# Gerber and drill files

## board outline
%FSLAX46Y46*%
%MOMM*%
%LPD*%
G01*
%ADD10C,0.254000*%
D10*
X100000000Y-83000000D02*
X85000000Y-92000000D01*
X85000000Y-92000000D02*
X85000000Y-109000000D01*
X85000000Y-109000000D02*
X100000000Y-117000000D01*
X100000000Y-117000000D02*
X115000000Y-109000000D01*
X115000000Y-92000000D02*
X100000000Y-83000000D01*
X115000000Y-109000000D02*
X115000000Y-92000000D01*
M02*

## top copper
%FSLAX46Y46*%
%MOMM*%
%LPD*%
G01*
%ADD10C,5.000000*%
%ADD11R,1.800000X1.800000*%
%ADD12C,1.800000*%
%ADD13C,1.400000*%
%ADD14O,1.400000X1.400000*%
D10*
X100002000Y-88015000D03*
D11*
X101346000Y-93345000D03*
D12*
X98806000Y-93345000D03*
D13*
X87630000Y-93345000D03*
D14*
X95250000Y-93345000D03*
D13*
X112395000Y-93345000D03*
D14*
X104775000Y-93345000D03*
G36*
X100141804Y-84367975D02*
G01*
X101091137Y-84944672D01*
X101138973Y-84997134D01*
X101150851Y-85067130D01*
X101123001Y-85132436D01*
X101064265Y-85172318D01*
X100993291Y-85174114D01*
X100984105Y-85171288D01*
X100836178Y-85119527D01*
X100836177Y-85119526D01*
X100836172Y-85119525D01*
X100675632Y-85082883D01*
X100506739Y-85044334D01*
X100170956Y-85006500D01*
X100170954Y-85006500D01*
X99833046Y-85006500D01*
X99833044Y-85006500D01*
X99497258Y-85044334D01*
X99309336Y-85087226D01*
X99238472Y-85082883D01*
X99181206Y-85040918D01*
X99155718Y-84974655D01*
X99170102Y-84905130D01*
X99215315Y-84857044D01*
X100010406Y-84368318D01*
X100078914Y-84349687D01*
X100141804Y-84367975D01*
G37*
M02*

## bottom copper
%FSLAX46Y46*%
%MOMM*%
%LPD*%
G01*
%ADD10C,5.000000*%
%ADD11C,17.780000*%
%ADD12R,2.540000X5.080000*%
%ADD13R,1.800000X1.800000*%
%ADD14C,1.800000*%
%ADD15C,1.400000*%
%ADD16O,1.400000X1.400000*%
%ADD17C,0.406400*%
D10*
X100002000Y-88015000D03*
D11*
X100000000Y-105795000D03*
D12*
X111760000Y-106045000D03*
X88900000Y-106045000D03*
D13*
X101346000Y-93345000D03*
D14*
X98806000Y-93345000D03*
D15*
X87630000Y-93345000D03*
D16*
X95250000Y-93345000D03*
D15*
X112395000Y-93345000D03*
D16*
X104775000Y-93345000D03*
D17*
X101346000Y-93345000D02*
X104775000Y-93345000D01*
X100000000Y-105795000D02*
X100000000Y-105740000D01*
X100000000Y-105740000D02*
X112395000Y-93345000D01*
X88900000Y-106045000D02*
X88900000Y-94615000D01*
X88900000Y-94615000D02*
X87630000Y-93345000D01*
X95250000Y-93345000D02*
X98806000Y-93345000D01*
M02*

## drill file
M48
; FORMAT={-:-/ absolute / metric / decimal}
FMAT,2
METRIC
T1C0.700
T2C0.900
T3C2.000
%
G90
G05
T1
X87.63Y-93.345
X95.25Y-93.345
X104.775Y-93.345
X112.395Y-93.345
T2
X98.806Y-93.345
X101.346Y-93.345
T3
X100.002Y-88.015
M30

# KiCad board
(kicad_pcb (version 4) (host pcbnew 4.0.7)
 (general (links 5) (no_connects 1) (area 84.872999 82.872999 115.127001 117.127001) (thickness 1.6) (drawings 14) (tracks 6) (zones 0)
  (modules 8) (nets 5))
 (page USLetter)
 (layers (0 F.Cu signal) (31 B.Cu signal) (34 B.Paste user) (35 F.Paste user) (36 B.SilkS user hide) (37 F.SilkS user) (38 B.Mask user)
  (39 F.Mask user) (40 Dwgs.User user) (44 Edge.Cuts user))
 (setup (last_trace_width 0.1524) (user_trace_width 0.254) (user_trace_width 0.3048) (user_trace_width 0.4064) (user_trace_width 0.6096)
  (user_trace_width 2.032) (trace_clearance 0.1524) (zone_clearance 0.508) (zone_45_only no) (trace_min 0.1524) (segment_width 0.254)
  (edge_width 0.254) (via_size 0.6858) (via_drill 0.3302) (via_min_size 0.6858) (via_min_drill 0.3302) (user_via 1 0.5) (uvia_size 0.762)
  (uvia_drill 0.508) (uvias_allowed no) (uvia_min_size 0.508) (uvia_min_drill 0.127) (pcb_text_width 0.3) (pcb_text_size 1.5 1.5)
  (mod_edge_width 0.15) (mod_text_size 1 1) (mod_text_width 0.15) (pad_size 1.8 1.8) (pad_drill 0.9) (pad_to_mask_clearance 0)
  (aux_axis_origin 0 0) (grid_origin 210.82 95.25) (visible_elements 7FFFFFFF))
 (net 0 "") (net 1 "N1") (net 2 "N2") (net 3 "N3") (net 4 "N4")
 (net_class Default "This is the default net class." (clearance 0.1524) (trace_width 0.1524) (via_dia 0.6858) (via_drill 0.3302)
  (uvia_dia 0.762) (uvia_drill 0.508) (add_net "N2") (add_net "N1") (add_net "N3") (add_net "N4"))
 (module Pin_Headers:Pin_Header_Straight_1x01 (layer F.Cu) (at 99.822 88.265)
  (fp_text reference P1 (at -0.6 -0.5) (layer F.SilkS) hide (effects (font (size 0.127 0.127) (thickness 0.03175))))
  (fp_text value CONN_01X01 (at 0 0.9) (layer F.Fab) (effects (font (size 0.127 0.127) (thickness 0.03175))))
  (pad "" thru_hole circle (at 0.18 -0.25) (size 5 5) (drill 2) (layers *.Cu B.Mask)))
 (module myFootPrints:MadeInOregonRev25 (layer F.Cu) (at 108.585 93.091)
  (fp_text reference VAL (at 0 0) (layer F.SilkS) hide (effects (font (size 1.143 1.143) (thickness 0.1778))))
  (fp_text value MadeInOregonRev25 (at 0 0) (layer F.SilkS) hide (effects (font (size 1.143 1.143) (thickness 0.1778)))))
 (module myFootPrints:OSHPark (layer F.Cu) (at 99.949 99.822)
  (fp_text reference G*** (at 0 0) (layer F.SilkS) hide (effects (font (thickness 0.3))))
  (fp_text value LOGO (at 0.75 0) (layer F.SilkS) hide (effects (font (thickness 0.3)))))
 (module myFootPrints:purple (layer F.Cu) (at 99.949 104.902)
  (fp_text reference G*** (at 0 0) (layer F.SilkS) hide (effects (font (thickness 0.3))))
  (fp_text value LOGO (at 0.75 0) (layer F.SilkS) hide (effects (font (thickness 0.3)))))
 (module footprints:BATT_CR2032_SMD (layer B.Cu) (at 100.33 106.045 180)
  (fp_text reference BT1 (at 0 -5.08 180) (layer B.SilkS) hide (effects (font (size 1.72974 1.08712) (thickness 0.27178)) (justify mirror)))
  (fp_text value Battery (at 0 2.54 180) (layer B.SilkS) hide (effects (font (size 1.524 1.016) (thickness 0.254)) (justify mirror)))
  (pad 2 smd circle (at 0.33 0.25 180) (size 17.78 17.78) (layers B.Cu B.Paste B.Mask) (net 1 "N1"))
  (pad 1 smd rect (at -11.43 0 180) (size 2.54 5.08) (layers B.Cu B.Paste B.Mask) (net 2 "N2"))
  (pad 1 smd rect (at 11.43 0 180) (size 2.54 5.08) (layers B.Cu B.Paste B.Mask) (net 2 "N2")))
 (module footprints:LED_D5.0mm (layer F.Cu) (at 101.346 93.345 180)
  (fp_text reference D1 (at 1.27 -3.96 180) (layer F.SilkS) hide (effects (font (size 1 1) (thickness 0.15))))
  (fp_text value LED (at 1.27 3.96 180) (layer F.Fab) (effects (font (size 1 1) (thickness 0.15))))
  (pad 1 thru_hole rect (at 0 0 180) (size 1.8 1.8) (drill 0.9) (layers *.Cu *.Mask) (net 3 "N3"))
  (pad 2 thru_hole circle (at 2.54 0 180) (size 1.8 1.8) (drill 0.9) (layers *.Cu *.Mask) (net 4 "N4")))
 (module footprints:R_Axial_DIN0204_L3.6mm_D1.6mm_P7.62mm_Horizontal (layer F.Cu) (at 87.63 93.345)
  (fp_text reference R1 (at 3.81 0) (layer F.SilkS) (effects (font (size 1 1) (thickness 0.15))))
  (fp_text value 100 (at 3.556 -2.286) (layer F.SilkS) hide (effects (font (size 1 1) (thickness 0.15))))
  (pad 1 thru_hole circle (at 0 0) (size 1.4 1.4) (drill 0.7) (layers *.Cu *.Mask) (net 2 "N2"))
  (pad 2 thru_hole oval (at 7.62 0) (size 1.4 1.4) (drill 0.7) (layers *.Cu *.Mask) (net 4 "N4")))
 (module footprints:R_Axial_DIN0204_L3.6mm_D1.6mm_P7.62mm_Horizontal (layer F.Cu) (at 112.395 93.345 180)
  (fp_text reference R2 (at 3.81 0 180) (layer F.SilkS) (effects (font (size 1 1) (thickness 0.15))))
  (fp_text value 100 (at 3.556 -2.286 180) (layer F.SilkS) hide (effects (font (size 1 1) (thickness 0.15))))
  (pad 1 thru_hole circle (at 0 0 180) (size 1.4 1.4) (drill 0.7) (layers *.Cu *.Mask) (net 1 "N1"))
  (pad 2 thru_hole oval (at 7.62 0 180) (size 1.4 1.4) (drill 0.7) (layers *.Cu *.Mask) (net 3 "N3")))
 (gr_line (start 100 83) (end 85 92) (angle 90) (layer Edge.Cuts) (width 0.254))
 (gr_line (start 85 92) (end 85 109) (angle 90) (layer Edge.Cuts) (width 0.254))
 (gr_line (start 85 109) (end 100 117) (angle 90) (layer Edge.Cuts) (width 0.254))
 (gr_line (start 100 117) (end 115 109) (angle 90) (layer Edge.Cuts) (width 0.254))
 (gr_line (start 115 92) (end 100 83) (angle 90) (layer Edge.Cuts) (width 0.254))
 (gr_line (start 115 109) (end 115 92) (angle 90) (layer Edge.Cuts) (width 0.254))
 (segment (start 101.346 93.345) (end 104.775 93.345) (width 0.4064) (layer B.Cu) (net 3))
 (segment (start 100 105.795) (end 100 105.74) (width 0.4064) (layer B.Cu) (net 1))
 (segment (start 100 105.74) (end 112.395 93.345) (width 0.4064) (layer B.Cu) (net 1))
 (segment (start 88.9 106.045) (end 88.9 94.615) (width 0.4064) (layer B.Cu) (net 2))
 (segment (start 88.9 94.615) (end 87.63 93.345) (width 0.4064) (layer B.Cu) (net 2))
 (segment (start 95.25 93.345) (end 98.806 93.345) (width 0.4064) (layer B.Cu) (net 4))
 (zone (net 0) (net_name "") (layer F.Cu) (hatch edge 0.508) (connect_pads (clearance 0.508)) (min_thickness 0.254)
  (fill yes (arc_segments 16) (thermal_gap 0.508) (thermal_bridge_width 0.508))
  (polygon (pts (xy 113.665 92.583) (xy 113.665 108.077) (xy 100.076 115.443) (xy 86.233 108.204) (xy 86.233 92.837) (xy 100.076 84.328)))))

